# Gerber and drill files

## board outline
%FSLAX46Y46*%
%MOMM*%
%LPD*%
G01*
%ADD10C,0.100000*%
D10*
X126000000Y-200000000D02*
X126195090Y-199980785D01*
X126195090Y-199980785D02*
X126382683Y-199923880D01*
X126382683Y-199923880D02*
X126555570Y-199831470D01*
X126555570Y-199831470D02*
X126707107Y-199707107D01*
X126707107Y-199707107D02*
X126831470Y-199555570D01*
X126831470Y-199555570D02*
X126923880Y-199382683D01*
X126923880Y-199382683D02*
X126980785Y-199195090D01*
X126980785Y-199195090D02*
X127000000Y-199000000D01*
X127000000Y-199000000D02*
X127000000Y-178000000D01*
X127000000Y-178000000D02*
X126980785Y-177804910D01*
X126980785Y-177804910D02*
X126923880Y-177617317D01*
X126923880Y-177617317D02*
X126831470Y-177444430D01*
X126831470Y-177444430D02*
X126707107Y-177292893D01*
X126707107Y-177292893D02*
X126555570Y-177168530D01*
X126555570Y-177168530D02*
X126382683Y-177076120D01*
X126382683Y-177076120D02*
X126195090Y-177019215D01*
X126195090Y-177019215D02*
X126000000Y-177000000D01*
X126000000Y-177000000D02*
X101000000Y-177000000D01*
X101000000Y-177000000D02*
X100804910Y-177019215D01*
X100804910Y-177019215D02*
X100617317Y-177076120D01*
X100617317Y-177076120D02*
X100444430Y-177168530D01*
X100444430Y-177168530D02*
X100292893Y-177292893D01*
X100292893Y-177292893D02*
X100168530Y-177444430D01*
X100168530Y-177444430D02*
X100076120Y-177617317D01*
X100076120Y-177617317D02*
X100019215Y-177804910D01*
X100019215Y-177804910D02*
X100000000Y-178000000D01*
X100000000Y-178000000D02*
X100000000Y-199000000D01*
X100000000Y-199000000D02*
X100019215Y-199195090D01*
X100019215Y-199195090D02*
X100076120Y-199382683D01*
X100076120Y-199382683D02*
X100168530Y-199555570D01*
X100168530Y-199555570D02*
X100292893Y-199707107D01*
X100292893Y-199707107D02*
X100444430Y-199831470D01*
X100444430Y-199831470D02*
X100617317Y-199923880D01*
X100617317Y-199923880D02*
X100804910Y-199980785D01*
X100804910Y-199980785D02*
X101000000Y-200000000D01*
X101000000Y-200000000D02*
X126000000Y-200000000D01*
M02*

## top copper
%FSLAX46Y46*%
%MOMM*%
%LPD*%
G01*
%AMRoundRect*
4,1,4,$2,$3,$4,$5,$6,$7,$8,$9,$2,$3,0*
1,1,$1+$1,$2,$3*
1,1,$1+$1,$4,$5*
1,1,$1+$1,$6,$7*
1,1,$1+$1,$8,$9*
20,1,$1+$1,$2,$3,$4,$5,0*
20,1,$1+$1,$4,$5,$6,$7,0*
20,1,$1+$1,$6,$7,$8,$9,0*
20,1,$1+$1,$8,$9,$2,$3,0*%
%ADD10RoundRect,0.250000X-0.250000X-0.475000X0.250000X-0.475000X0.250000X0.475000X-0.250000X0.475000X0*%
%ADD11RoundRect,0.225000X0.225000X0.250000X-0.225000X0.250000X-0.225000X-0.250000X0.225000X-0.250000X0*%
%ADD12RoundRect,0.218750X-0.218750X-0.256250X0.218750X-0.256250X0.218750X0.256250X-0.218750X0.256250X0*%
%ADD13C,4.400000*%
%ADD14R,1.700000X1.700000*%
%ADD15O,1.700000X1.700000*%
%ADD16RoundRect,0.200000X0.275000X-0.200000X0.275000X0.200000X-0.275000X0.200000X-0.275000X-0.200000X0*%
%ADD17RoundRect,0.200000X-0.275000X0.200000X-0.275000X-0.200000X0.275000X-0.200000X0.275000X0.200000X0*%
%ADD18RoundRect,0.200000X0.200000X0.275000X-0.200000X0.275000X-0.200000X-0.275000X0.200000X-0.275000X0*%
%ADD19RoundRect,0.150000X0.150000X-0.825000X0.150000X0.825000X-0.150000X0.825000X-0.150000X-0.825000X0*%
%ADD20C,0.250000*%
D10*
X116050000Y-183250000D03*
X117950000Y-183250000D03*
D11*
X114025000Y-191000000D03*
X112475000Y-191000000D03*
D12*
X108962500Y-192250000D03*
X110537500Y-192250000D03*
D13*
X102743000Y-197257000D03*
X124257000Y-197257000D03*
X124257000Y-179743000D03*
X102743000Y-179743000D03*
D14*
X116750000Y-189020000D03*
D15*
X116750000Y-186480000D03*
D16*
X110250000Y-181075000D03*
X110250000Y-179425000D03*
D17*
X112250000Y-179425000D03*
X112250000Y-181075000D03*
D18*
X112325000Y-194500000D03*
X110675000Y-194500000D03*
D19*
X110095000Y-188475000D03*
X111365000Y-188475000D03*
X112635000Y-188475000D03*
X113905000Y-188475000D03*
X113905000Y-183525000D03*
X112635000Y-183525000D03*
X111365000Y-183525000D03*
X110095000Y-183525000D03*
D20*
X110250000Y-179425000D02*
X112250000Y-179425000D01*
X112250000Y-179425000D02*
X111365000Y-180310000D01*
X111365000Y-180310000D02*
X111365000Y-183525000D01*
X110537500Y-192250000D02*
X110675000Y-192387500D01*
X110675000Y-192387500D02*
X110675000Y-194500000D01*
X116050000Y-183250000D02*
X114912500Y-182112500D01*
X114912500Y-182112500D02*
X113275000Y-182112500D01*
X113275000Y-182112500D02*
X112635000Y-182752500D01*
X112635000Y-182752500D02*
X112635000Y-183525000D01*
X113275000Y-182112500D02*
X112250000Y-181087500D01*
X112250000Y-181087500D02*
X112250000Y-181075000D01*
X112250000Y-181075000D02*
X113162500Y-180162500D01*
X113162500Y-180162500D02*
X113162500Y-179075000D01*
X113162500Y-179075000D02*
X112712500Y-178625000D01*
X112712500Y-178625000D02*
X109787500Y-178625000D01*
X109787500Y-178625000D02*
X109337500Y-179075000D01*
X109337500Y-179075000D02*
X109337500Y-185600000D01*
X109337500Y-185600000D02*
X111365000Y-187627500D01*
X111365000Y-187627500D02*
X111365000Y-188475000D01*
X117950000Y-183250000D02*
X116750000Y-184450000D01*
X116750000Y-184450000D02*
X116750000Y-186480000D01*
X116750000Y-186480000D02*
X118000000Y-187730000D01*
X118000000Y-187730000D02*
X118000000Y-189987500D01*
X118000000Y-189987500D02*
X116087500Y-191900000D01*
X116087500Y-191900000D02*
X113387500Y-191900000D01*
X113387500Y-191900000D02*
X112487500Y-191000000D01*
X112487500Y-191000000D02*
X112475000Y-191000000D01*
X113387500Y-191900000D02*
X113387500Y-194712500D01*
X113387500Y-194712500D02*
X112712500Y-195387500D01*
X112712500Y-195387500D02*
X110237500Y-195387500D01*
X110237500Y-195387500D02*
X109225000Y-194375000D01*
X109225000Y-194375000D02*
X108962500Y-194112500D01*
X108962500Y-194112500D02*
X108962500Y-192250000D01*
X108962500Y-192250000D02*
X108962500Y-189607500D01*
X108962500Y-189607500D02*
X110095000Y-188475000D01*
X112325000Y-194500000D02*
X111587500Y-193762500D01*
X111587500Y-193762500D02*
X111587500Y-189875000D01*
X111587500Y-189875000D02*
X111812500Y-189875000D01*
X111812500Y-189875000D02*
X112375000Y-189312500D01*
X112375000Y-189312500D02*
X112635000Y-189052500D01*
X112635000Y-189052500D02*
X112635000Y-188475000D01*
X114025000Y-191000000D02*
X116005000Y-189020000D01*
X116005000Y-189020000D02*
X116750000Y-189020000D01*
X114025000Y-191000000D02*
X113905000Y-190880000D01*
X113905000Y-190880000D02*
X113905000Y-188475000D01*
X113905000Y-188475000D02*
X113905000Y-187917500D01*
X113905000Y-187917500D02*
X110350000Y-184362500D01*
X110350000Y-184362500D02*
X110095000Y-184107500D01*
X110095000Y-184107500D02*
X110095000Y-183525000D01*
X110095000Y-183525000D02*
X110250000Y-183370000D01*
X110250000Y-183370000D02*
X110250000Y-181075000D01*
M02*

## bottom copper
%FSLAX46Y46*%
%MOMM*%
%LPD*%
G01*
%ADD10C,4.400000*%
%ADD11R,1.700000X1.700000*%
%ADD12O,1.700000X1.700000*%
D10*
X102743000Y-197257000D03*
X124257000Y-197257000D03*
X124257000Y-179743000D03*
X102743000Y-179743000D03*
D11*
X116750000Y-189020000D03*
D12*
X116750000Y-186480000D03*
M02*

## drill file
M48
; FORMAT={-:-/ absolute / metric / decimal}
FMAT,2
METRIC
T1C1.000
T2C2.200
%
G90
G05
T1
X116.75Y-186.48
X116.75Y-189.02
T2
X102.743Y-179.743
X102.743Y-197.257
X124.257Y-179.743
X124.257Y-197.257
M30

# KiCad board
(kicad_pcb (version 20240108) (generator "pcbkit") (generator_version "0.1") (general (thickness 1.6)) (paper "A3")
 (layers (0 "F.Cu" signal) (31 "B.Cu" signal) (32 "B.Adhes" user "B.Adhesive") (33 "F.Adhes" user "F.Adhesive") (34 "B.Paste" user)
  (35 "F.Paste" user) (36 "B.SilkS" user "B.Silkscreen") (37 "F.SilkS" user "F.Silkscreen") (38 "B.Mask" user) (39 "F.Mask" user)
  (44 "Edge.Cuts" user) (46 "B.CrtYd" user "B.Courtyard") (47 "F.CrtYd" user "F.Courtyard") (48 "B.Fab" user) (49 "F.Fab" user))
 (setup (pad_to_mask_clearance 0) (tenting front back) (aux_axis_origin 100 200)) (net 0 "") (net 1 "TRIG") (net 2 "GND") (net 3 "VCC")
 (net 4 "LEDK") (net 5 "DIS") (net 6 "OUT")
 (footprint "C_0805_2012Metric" (layer "F.Cu") (at 117 183.25 0)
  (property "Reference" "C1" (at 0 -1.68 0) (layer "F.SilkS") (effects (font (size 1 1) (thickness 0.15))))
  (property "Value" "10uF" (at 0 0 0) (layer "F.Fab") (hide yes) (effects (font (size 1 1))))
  (pad "1" smd roundrect (at -0.95 0 0) (size 1 1.45) (layers "F.Cu" "F.Paste" "F.Mask") (roundrect_rratio 0.250000000000)
   (solder_mask_margin 0.05) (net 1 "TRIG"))
  (pad "2" smd roundrect (at 0.95 0 0) (size 1 1.45) (layers "F.Cu" "F.Paste" "F.Mask") (roundrect_rratio 0.250000000000)
   (solder_mask_margin 0.05) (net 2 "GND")))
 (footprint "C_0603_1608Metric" (layer "F.Cu") (at 113.25 191 180)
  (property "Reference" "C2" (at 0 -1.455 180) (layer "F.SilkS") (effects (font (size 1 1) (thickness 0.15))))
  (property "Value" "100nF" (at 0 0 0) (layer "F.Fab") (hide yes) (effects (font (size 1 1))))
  (pad "1" smd roundrect (at -0.775 0 180) (size 0.9 0.95) (layers "F.Cu" "F.Paste" "F.Mask") (roundrect_rratio 0.250000000000)
   (solder_mask_margin 0.05) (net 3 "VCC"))
  (pad "2" smd roundrect (at 0.775 0 180) (size 0.9 0.95) (layers "F.Cu" "F.Paste" "F.Mask") (roundrect_rratio 0.250000000000)
   (solder_mask_margin 0.05) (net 2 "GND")))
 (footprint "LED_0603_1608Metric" (layer "F.Cu") (at 109.75 192.25 0)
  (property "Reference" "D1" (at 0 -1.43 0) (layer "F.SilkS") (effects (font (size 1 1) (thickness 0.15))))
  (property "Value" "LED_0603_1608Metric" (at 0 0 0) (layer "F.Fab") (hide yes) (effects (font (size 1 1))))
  (pad "1" smd roundrect (at -0.7875 0 0) (size 0.875 0.95) (layers "F.Cu" "F.Paste" "F.Mask") (roundrect_rratio 0.250000000000)
   (solder_mask_margin 0.05) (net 2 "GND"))
  (pad "2" smd roundrect (at 0.7875 0 0) (size 0.875 0.95) (layers "F.Cu" "F.Paste" "F.Mask") (roundrect_rratio 0.250000000000)
   (solder_mask_margin 0.05) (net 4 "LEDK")))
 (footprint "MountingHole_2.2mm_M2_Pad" (layer "F.Cu") (at 102.743 197.257 0)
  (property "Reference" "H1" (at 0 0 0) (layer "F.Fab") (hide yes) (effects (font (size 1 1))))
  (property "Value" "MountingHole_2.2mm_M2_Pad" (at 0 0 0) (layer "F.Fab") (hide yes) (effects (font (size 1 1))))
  (pad "1" thru_hole circle (at 0 0 0) (size 4.4 4.4) (drill 2.2) (layers "*.Cu" "*.Mask") (solder_mask_margin 0.05)))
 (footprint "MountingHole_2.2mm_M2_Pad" (layer "F.Cu") (at 124.257 197.257 0)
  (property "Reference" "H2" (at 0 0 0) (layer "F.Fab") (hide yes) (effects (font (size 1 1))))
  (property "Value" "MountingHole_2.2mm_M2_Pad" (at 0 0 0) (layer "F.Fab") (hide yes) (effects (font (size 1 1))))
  (pad "1" thru_hole circle (at 0 0 0) (size 4.4 4.4) (drill 2.2) (layers "*.Cu" "*.Mask") (solder_mask_margin 0.05)))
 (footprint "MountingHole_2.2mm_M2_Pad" (layer "F.Cu") (at 124.257 179.743 0)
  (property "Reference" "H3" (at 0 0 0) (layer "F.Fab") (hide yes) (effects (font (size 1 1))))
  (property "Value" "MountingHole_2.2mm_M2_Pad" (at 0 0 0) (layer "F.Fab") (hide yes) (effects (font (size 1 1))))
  (pad "1" thru_hole circle (at 0 0 0) (size 4.4 4.4) (drill 2.2) (layers "*.Cu" "*.Mask") (solder_mask_margin 0.05)))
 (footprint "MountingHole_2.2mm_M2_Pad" (layer "F.Cu") (at 102.743 179.743 0)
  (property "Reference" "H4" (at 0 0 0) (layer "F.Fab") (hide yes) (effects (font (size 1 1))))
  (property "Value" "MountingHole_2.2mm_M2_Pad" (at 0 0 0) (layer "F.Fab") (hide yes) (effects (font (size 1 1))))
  (pad "1" thru_hole circle (at 0 0 0) (size 4.4 4.4) (drill 2.2) (layers "*.Cu" "*.Mask") (solder_mask_margin 0.05)))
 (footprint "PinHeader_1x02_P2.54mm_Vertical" (layer "F.Cu") (at 116.75 187.75 180)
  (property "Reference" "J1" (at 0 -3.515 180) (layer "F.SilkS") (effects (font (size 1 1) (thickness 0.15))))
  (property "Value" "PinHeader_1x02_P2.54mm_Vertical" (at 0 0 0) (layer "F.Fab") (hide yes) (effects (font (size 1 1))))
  (pad "1" thru_hole rect (at 0 -1.27 180) (size 1.7 1.7) (drill 1) (layers "*.Cu" "*.Mask") (solder_mask_margin 0.05) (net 3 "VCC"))
  (pad "2" thru_hole oval (at 0 1.27 180) (size 1.7 1.7) (drill 1) (layers "*.Cu" "*.Mask") (solder_mask_margin 0.05) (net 2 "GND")))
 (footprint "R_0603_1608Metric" (layer "F.Cu") (at 110.25 180.25 90)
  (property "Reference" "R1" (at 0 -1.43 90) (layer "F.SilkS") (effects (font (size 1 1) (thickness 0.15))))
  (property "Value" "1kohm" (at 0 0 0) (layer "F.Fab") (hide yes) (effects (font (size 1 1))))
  (pad "1" smd roundrect (at -0.825 0 90) (size 0.8 0.95) (layers "F.Cu" "F.Paste" "F.Mask") (roundrect_rratio 0.250000000000)
   (solder_mask_margin 0.05) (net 3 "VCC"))
  (pad "2" smd roundrect (at 0.825 0 90) (size 0.8 0.95) (layers "F.Cu" "F.Paste" "F.Mask") (roundrect_rratio 0.250000000000)
   (solder_mask_margin 0.05) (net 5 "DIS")))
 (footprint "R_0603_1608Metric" (layer "F.Cu") (at 112.25 180.25 270)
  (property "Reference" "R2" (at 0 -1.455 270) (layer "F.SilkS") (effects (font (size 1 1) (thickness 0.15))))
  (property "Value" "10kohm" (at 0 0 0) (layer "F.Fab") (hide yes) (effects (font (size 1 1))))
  (pad "1" smd roundrect (at -0.825 0 270) (size 0.8 0.95) (layers "F.Cu" "F.Paste" "F.Mask") (roundrect_rratio 0.250000000000)
   (solder_mask_margin 0.05) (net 5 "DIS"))
  (pad "2" smd roundrect (at 0.825 0 270) (size 0.8 0.95) (layers "F.Cu" "F.Paste" "F.Mask") (roundrect_rratio 0.250000000000)
   (solder_mask_margin 0.05) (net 1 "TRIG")))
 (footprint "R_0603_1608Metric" (layer "F.Cu") (at 111.5 194.5 180)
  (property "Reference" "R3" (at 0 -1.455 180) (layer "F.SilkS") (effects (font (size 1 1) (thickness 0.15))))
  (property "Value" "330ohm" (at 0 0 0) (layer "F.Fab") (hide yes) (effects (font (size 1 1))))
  (pad "1" smd roundrect (at -0.825 0 180) (size 0.8 0.95) (layers "F.Cu" "F.Paste" "F.Mask") (roundrect_rratio 0.250000000000)
   (solder_mask_margin 0.05) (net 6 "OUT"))
  (pad "2" smd roundrect (at 0.825 0 180) (size 0.8 0.95) (layers "F.Cu" "F.Paste" "F.Mask") (roundrect_rratio 0.250000000000)
   (solder_mask_margin 0.05) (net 4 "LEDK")))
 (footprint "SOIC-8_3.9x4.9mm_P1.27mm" (layer "F.Cu") (at 112 186 90)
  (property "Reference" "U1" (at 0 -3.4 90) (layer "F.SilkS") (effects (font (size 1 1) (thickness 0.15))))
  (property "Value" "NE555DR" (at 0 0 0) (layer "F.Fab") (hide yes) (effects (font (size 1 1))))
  (pad "1" smd roundrect (at -2.475 -1.905 90) (size 1.95 0.6) (layers "F.Cu" "F.Paste" "F.Mask") (roundrect_rratio 0.250000000000)
   (solder_mask_margin 0.05) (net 2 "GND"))
  (pad "2" smd roundrect (at -2.475 -0.635 90) (size 1.95 0.6) (layers "F.Cu" "F.Paste" "F.Mask") (roundrect_rratio 0.250000000000)
   (solder_mask_margin 0.05) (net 1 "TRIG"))
  (pad "3" smd roundrect (at -2.475 0.635 90) (size 1.95 0.6) (layers "F.Cu" "F.Paste" "F.Mask") (roundrect_rratio 0.250000000000)
   (solder_mask_margin 0.05) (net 6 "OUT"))
  (pad "4" smd roundrect (at -2.475 1.905 90) (size 1.95 0.6) (layers "F.Cu" "F.Paste" "F.Mask") (roundrect_rratio 0.250000000000)
   (solder_mask_margin 0.05) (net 3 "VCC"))
  (pad "5" smd roundrect (at 2.475 1.905 90) (size 1.95 0.6) (layers "F.Cu" "F.Paste" "F.Mask") (roundrect_rratio 0.250000000000)
   (solder_mask_margin 0.05))
  (pad "6" smd roundrect (at 2.475 0.635 90) (size 1.95 0.6) (layers "F.Cu" "F.Paste" "F.Mask") (roundrect_rratio 0.250000000000)
   (solder_mask_margin 0.05) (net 1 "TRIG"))
  (pad "7" smd roundrect (at 2.475 -0.635 90) (size 1.95 0.6) (layers "F.Cu" "F.Paste" "F.Mask") (roundrect_rratio 0.250000000000)
   (solder_mask_margin 0.05) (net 5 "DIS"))
  (pad "8" smd roundrect (at 2.475 -1.905 90) (size 1.95 0.6) (layers "F.Cu" "F.Paste" "F.Mask") (roundrect_rratio 0.250000000000)
   (solder_mask_margin 0.05) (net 3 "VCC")))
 (gr_line (start 126 200) (end 126.19509 199.980785) (stroke (width 0.1) (type solid)) (layer "Edge.Cuts"))
 (gr_line (start 126.19509 199.980785) (end 126.382683 199.92388) (stroke (width 0.1) (type solid)) (layer "Edge.Cuts"))
 (gr_line (start 126.382683 199.92388) (end 126.55557 199.83147) (stroke (width 0.1) (type solid)) (layer "Edge.Cuts"))
 (gr_line (start 126.55557 199.83147) (end 126.707107 199.707107) (stroke (width 0.1) (type solid)) (layer "Edge.Cuts"))
 (gr_line (start 126.707107 199.707107) (end 126.83147 199.55557) (stroke (width 0.1) (type solid)) (layer "Edge.Cuts"))
 (gr_line (start 126.83147 199.55557) (end 126.92388 199.382683) (stroke (width 0.1) (type solid)) (layer "Edge.Cuts"))
 (gr_line (start 126.92388 199.382683) (end 126.980785 199.19509) (stroke (width 0.1) (type solid)) (layer "Edge.Cuts"))
 (gr_line (start 126.980785 199.19509) (end 127 199) (stroke (width 0.1) (type solid)) (layer "Edge.Cuts"))
 (gr_line (start 127 199) (end 127 178) (stroke (width 0.1) (type solid)) (layer "Edge.Cuts"))
 (gr_line (start 127 178) (end 126.980785 177.80491) (stroke (width 0.1) (type solid)) (layer "Edge.Cuts"))
 (gr_line (start 126.980785 177.80491) (end 126.92388 177.617317) (stroke (width 0.1) (type solid)) (layer "Edge.Cuts"))
 (gr_line (start 126.92388 177.617317) (end 126.83147 177.44443) (stroke (width 0.1) (type solid)) (layer "Edge.Cuts"))
 (gr_line (start 126.83147 177.44443) (end 126.707107 177.292893) (stroke (width 0.1) (type solid)) (layer "Edge.Cuts"))
 (gr_line (start 126.707107 177.292893) (end 126.55557 177.16853) (stroke (width 0.1) (type solid)) (layer "Edge.Cuts"))
 (gr_line (start 126.55557 177.16853) (end 126.382683 177.07612) (stroke (width 0.1) (type solid)) (layer "Edge.Cuts"))
 (gr_line (start 126.382683 177.07612) (end 126.19509 177.019215) (stroke (width 0.1) (type solid)) (layer "Edge.Cuts"))
 (gr_line (start 126.19509 177.019215) (end 126 177) (stroke (width 0.1) (type solid)) (layer "Edge.Cuts"))
 (gr_line (start 126 177) (end 101 177) (stroke (width 0.1) (type solid)) (layer "Edge.Cuts"))
 (gr_line (start 101 177) (end 100.80491 177.019215) (stroke (width 0.1) (type solid)) (layer "Edge.Cuts"))
 (gr_line (start 100.80491 177.019215) (end 100.617317 177.07612) (stroke (width 0.1) (type solid)) (layer "Edge.Cuts"))
 (gr_line (start 100.617317 177.07612) (end 100.44443 177.16853) (stroke (width 0.1) (type solid)) (layer "Edge.Cuts"))
 (gr_line (start 100.44443 177.16853) (end 100.292893 177.292893) (stroke (width 0.1) (type solid)) (layer "Edge.Cuts"))
 (gr_line (start 100.292893 177.292893) (end 100.16853 177.44443) (stroke (width 0.1) (type solid)) (layer "Edge.Cuts"))
 (gr_line (start 100.16853 177.44443) (end 100.07612 177.617317) (stroke (width 0.1) (type solid)) (layer "Edge.Cuts"))
 (gr_line (start 100.07612 177.617317) (end 100.019215 177.80491) (stroke (width 0.1) (type solid)) (layer "Edge.Cuts"))
 (gr_line (start 100.019215 177.80491) (end 100 178) (stroke (width 0.1) (type solid)) (layer "Edge.Cuts"))
 (gr_line (start 100 178) (end 100 199) (stroke (width 0.1) (type solid)) (layer "Edge.Cuts"))
 (gr_line (start 100 199) (end 100.019215 199.19509) (stroke (width 0.1) (type solid)) (layer "Edge.Cuts"))
 (gr_line (start 100.019215 199.19509) (end 100.07612 199.382683) (stroke (width 0.1) (type solid)) (layer "Edge.Cuts"))
 (gr_line (start 100.07612 199.382683) (end 100.16853 199.55557) (stroke (width 0.1) (type solid)) (layer "Edge.Cuts"))
 (gr_line (start 100.16853 199.55557) (end 100.292893 199.707107) (stroke (width 0.1) (type solid)) (layer "Edge.Cuts"))
 (gr_line (start 100.292893 199.707107) (end 100.44443 199.83147) (stroke (width 0.1) (type solid)) (layer "Edge.Cuts"))
 (gr_line (start 100.44443 199.83147) (end 100.617317 199.92388) (stroke (width 0.1) (type solid)) (layer "Edge.Cuts"))
 (gr_line (start 100.617317 199.92388) (end 100.80491 199.980785) (stroke (width 0.1) (type solid)) (layer "Edge.Cuts"))
 (gr_line (start 100.80491 199.980785) (end 101 200) (stroke (width 0.1) (type solid)) (layer "Edge.Cuts"))
 (gr_line (start 101 200) (end 126 200) (stroke (width 0.1) (type solid)) (layer "Edge.Cuts"))
 (segment (start 110.25 179.425) (end 112.25 179.425) (width 0.25) (layer "F.Cu") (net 5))
 (segment (start 112.25 179.425) (end 111.365 180.31) (width 0.25) (layer "F.Cu") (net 5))
 (segment (start 111.365 180.31) (end 111.365 183.525) (width 0.25) (layer "F.Cu") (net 5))
 (segment (start 110.5375 192.25) (end 110.675 192.3875) (width 0.25) (layer "F.Cu") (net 4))
 (segment (start 110.675 192.3875) (end 110.675 194.5) (width 0.25) (layer "F.Cu") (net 4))
 (segment (start 116.05 183.25) (end 114.9125 182.1125) (width 0.25) (layer "F.Cu") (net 1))
 (segment (start 114.9125 182.1125) (end 113.275 182.1125) (width 0.25) (layer "F.Cu") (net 1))
 (segment (start 113.275 182.1125) (end 112.635 182.7525) (width 0.25) (layer "F.Cu") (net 1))
 (segment (start 112.635 182.7525) (end 112.635 183.525) (width 0.25) (layer "F.Cu") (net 1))
 (segment (start 113.275 182.1125) (end 112.25 181.0875) (width 0.25) (layer "F.Cu") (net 1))
 (segment (start 112.25 181.0875) (end 112.25 181.075) (width 0.25) (layer "F.Cu") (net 1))
 (segment (start 112.25 181.075) (end 113.1625 180.1625) (width 0.25) (layer "F.Cu") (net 1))
 (segment (start 113.1625 180.1625) (end 113.1625 179.075) (width 0.25) (layer "F.Cu") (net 1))
 (segment (start 113.1625 179.075) (end 112.7125 178.625) (width 0.25) (layer "F.Cu") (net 1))
 (segment (start 112.7125 178.625) (end 109.7875 178.625) (width 0.25) (layer "F.Cu") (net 1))
 (segment (start 109.7875 178.625) (end 109.3375 179.075) (width 0.25) (layer "F.Cu") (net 1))
 (segment (start 109.3375 179.075) (end 109.3375 185.6) (width 0.25) (layer "F.Cu") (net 1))
 (segment (start 109.3375 185.6) (end 111.365 187.6275) (width 0.25) (layer "F.Cu") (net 1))
 (segment (start 111.365 187.6275) (end 111.365 188.475) (width 0.25) (layer "F.Cu") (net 1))
 (segment (start 117.95 183.25) (end 116.75 184.45) (width 0.25) (layer "F.Cu") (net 2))
 (segment (start 116.75 184.45) (end 116.75 186.48) (width 0.25) (layer "F.Cu") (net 2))
 (segment (start 116.75 186.48) (end 118 187.73) (width 0.25) (layer "F.Cu") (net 2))
 (segment (start 118 187.73) (end 118 189.9875) (width 0.25) (layer "F.Cu") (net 2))
 (segment (start 118 189.9875) (end 116.0875 191.9) (width 0.25) (layer "F.Cu") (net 2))
 (segment (start 116.0875 191.9) (end 113.3875 191.9) (width 0.25) (layer "F.Cu") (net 2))
 (segment (start 113.3875 191.9) (end 112.4875 191) (width 0.25) (layer "F.Cu") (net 2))
 (segment (start 112.4875 191) (end 112.475 191) (width 0.25) (layer "F.Cu") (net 2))
 (segment (start 113.3875 191.9) (end 113.3875 194.7125) (width 0.25) (layer "F.Cu") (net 2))
 (segment (start 113.3875 194.7125) (end 112.7125 195.3875) (width 0.25) (layer "F.Cu") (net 2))
 (segment (start 112.7125 195.3875) (end 110.2375 195.3875) (width 0.25) (layer "F.Cu") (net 2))
 (segment (start 110.2375 195.3875) (end 109.225 194.375) (width 0.25) (layer "F.Cu") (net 2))
 (segment (start 109.225 194.375) (end 108.9625 194.1125) (width 0.25) (layer "F.Cu") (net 2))
 (segment (start 108.9625 194.1125) (end 108.9625 192.25) (width 0.25) (layer "F.Cu") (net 2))
 (segment (start 108.9625 192.25) (end 108.9625 189.6075) (width 0.25) (layer "F.Cu") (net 2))
 (segment (start 108.9625 189.6075) (end 110.095 188.475) (width 0.25) (layer "F.Cu") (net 2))
 (segment (start 112.325 194.5) (end 111.5875 193.7625) (width 0.25) (layer "F.Cu") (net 6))
 (segment (start 111.5875 193.7625) (end 111.5875 189.875) (width 0.25) (layer "F.Cu") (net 6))
 (segment (start 111.5875 189.875) (end 111.8125 189.875) (width 0.25) (layer "F.Cu") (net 6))
 (segment (start 111.8125 189.875) (end 112.375 189.3125) (width 0.25) (layer "F.Cu") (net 6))
 (segment (start 112.375 189.3125) (end 112.635 189.0525) (width 0.25) (layer "F.Cu") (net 6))
 (segment (start 112.635 189.0525) (end 112.635 188.475) (width 0.25) (layer "F.Cu") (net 6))
 (segment (start 114.025 191) (end 116.005 189.02) (width 0.25) (layer "F.Cu") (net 3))
 (segment (start 116.005 189.02) (end 116.75 189.02) (width 0.25) (layer "F.Cu") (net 3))
 (segment (start 114.025 191) (end 113.905 190.88) (width 0.25) (layer "F.Cu") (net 3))
 (segment (start 113.905 190.88) (end 113.905 188.475) (width 0.25) (layer "F.Cu") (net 3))
 (segment (start 113.905 188.475) (end 113.905 187.9175) (width 0.25) (layer "F.Cu") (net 3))
 (segment (start 113.905 187.9175) (end 110.35 184.3625) (width 0.25) (layer "F.Cu") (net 3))
 (segment (start 110.35 184.3625) (end 110.095 184.1075) (width 0.25) (layer "F.Cu") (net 3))
 (segment (start 110.095 184.1075) (end 110.095 183.525) (width 0.25) (layer "F.Cu") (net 3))
 (segment (start 110.095 183.525) (end 110.25 183.37) (width 0.25) (layer "F.Cu") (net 3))
 (segment (start 110.25 183.37) (end 110.25 181.075) (width 0.25) (layer "F.Cu") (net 3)))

